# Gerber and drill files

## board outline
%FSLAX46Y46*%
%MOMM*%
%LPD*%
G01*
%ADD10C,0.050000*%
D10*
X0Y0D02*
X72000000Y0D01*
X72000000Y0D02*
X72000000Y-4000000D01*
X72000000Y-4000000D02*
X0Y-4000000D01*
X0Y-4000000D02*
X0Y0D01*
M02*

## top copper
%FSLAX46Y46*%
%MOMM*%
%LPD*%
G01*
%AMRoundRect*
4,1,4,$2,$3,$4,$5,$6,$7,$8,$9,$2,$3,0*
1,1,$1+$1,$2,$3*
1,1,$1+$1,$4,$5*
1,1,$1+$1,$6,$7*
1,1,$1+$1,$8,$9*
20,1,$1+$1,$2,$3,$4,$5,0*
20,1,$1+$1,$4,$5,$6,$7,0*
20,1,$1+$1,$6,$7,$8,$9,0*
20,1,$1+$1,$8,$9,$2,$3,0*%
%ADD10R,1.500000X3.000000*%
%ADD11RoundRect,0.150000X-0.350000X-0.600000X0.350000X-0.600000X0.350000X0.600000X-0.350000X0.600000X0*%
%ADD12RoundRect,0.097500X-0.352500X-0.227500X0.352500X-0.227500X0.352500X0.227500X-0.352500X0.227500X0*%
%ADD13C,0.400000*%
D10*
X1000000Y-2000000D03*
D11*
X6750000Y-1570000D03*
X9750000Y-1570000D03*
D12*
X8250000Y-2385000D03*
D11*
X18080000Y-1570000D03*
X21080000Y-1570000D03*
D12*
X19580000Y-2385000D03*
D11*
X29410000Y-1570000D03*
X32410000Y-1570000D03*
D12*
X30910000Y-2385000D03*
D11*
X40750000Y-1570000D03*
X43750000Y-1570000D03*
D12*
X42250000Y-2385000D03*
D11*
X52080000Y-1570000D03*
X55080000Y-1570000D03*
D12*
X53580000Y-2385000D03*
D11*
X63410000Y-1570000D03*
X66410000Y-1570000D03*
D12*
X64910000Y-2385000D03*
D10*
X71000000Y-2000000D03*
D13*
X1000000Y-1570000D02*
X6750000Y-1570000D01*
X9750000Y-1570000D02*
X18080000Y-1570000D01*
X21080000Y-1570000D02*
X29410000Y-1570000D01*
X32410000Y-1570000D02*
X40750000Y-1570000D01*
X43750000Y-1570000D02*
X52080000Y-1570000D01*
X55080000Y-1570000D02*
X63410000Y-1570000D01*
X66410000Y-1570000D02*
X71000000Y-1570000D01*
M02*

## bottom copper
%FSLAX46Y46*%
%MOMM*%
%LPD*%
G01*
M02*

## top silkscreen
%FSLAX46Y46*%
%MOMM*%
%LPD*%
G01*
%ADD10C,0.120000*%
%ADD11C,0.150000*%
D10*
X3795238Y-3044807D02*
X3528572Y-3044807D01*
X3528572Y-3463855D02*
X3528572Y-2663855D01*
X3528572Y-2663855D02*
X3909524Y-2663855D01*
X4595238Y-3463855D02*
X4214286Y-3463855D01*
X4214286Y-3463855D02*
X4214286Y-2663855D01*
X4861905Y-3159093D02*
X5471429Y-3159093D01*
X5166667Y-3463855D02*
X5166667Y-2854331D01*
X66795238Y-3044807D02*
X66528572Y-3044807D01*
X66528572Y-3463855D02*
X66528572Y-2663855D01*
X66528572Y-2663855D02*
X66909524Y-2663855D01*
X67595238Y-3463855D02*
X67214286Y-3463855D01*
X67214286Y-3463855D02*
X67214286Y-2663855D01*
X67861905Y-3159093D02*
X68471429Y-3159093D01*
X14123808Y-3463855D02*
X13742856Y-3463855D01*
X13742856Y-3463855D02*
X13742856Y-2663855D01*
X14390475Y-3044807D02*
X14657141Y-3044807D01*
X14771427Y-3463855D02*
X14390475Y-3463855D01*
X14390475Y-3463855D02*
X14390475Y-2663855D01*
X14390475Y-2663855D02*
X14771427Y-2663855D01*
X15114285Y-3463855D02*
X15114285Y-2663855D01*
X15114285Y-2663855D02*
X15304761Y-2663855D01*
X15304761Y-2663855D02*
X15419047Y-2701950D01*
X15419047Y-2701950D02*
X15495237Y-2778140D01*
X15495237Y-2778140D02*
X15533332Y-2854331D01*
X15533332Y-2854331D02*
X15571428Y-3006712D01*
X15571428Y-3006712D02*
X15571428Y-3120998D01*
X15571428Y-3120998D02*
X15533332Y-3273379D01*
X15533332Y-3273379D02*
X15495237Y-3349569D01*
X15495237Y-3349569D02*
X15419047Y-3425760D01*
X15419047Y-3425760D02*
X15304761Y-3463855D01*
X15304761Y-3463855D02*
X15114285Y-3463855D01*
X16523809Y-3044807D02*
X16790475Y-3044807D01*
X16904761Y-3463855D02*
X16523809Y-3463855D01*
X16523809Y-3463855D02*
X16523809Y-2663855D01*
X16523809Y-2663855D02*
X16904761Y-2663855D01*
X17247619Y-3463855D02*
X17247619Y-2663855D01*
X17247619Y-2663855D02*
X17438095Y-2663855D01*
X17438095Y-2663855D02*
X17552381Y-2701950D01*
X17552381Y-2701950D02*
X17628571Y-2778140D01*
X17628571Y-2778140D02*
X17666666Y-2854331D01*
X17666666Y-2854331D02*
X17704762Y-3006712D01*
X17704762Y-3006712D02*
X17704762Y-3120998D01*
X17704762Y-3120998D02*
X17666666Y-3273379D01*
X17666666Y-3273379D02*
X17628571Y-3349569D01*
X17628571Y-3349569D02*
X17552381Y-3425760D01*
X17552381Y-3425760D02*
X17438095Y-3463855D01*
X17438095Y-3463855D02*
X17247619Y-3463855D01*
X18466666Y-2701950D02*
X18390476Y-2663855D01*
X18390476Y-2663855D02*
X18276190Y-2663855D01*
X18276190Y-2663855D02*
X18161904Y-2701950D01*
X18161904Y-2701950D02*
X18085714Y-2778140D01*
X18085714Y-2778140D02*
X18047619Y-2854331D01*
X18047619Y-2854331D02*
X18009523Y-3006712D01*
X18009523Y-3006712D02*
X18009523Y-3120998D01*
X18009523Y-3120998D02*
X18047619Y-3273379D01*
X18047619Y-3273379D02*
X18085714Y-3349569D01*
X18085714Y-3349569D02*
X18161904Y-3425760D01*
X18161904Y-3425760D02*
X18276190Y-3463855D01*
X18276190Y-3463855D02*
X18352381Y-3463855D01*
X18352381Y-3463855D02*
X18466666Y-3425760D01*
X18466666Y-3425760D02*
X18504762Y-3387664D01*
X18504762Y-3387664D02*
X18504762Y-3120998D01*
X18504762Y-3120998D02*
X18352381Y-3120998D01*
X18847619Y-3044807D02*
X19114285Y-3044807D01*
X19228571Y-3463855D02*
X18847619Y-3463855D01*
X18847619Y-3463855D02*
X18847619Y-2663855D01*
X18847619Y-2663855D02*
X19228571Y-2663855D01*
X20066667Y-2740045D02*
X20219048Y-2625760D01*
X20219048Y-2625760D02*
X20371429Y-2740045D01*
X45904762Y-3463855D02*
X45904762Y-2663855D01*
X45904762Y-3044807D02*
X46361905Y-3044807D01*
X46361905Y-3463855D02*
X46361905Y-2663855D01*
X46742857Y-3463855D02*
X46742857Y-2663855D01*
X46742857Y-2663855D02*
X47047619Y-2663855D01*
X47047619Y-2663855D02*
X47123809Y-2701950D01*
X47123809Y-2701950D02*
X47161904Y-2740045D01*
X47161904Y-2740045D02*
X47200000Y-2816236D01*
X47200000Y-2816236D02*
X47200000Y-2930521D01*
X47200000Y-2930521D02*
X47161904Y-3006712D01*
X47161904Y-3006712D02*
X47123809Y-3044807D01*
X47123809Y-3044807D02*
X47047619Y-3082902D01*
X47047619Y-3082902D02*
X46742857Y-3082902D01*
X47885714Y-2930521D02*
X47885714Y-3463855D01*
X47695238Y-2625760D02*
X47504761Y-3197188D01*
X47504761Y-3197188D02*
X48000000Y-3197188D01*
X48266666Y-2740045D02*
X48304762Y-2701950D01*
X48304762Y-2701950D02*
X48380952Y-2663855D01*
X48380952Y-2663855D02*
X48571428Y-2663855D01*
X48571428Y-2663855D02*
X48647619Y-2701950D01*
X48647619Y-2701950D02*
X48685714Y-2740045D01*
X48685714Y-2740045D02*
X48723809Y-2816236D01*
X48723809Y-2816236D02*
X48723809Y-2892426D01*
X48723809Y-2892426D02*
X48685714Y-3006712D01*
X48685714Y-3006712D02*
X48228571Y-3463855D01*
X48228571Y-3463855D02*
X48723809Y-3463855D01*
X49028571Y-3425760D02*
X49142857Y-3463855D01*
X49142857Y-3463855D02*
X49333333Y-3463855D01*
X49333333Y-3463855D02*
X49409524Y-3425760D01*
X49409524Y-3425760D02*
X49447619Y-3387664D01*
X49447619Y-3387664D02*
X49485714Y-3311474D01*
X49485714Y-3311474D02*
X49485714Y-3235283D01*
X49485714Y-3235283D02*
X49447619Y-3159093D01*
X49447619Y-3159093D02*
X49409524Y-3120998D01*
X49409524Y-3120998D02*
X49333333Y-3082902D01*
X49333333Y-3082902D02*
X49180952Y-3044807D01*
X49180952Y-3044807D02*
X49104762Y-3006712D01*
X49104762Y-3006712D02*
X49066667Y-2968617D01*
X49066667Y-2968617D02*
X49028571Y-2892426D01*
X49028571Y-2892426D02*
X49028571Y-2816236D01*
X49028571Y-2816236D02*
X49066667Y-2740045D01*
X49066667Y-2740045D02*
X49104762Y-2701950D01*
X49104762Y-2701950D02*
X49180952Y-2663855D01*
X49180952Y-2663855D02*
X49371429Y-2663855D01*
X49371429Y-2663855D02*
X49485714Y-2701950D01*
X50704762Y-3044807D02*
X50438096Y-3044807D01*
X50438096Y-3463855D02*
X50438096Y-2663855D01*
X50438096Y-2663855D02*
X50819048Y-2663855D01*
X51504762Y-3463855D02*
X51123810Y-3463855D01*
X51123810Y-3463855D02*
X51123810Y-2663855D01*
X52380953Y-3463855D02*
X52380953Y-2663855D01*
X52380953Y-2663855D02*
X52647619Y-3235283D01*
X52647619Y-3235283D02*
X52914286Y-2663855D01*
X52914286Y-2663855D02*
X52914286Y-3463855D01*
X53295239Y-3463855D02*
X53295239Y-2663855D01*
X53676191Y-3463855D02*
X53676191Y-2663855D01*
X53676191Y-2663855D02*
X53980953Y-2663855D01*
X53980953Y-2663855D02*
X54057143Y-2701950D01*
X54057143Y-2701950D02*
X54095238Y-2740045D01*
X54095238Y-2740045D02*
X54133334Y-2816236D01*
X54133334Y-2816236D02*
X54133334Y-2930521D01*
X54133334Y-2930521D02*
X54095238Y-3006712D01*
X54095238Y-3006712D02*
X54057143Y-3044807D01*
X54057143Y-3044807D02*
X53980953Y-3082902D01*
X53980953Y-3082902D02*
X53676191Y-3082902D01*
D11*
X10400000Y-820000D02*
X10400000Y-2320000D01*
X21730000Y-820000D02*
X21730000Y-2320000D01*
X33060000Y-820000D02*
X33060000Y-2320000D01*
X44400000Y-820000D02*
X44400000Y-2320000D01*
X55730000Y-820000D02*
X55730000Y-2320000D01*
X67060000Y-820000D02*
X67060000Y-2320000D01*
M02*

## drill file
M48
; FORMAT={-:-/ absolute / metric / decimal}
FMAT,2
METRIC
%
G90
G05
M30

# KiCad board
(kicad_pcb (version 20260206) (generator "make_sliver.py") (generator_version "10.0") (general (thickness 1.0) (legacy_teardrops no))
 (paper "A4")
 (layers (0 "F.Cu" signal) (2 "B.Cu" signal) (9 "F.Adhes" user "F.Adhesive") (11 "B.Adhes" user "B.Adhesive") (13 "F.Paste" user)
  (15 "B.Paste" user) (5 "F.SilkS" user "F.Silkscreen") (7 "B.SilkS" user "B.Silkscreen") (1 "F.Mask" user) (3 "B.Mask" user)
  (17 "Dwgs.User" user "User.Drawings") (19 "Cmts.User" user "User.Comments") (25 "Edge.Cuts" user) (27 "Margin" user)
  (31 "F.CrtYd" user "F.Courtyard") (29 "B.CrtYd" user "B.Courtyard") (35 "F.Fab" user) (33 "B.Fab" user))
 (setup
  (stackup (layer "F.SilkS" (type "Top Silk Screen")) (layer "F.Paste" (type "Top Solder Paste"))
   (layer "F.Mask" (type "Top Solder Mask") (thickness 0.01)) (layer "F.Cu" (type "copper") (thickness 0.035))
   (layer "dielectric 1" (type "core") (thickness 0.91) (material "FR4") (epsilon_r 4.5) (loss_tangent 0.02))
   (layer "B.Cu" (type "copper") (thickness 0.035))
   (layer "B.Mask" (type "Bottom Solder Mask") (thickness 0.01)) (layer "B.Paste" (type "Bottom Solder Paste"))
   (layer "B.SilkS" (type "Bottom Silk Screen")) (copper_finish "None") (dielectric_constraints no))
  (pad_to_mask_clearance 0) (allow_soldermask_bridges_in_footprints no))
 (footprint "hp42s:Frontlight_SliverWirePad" (layer "F.Cu") (at 1 2)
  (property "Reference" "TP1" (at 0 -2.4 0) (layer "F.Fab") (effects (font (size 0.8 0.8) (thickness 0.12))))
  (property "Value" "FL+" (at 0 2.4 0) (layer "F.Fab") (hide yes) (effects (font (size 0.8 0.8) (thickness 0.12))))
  (pad "1" smd rect (at 0 0) (size 1.5 3) (layers "F.Cu" "F.Mask") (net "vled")))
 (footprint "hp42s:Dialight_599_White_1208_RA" (layer "F.Cu") (at 8.25 1.57)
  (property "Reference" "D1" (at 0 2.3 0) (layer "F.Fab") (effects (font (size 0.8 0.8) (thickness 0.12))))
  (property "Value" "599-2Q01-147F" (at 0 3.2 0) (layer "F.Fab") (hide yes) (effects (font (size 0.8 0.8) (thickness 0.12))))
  (fp_line (start 2.15 -0.75) (end 2.15 0.75) (stroke (width 0.15) (type solid)) (layer "F.SilkS"))
  (pad "2" smd roundrect (at -1.5 0) (size 1 1.5) (layers "F.Cu" "F.Paste" "F.Mask") (roundrect_rratio 0.15) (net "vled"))
  (pad "1" smd roundrect (at 1.5 0) (size 1 1.5) (layers "F.Cu" "F.Paste" "F.Mask") (roundrect_rratio 0.15) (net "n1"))
  (pad "3" smd roundrect (at 0 0.815) (size 0.9 0.65) (layers "F.Cu" "F.Paste" "F.Mask") (roundrect_rratio 0.15)))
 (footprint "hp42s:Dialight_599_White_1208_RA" (layer "F.Cu") (at 19.58 1.57)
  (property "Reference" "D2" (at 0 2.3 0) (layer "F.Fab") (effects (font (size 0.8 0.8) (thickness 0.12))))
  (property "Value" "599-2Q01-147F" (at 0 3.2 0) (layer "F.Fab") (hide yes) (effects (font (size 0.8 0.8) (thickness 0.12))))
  (fp_line (start 2.15 -0.75) (end 2.15 0.75) (stroke (width 0.15) (type solid)) (layer "F.SilkS"))
  (pad "2" smd roundrect (at -1.5 0) (size 1 1.5) (layers "F.Cu" "F.Paste" "F.Mask") (roundrect_rratio 0.15) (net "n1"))
  (pad "1" smd roundrect (at 1.5 0) (size 1 1.5) (layers "F.Cu" "F.Paste" "F.Mask") (roundrect_rratio 0.15) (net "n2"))
  (pad "3" smd roundrect (at 0 0.815) (size 0.9 0.65) (layers "F.Cu" "F.Paste" "F.Mask") (roundrect_rratio 0.15)))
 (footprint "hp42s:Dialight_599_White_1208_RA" (layer "F.Cu") (at 30.91 1.57)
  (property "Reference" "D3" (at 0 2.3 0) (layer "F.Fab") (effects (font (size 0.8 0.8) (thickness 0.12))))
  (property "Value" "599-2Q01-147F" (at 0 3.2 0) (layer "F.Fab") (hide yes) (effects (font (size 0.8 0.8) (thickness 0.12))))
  (fp_line (start 2.15 -0.75) (end 2.15 0.75) (stroke (width 0.15) (type solid)) (layer "F.SilkS"))
  (pad "2" smd roundrect (at -1.5 0) (size 1 1.5) (layers "F.Cu" "F.Paste" "F.Mask") (roundrect_rratio 0.15) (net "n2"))
  (pad "1" smd roundrect (at 1.5 0) (size 1 1.5) (layers "F.Cu" "F.Paste" "F.Mask") (roundrect_rratio 0.15) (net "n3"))
  (pad "3" smd roundrect (at 0 0.815) (size 0.9 0.65) (layers "F.Cu" "F.Paste" "F.Mask") (roundrect_rratio 0.15)))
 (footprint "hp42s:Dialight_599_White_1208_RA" (layer "F.Cu") (at 42.25 1.57)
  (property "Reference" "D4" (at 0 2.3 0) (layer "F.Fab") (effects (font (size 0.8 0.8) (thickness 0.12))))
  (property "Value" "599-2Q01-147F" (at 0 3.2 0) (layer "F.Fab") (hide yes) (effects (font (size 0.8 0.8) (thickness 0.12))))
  (fp_line (start 2.15 -0.75) (end 2.15 0.75) (stroke (width 0.15) (type solid)) (layer "F.SilkS"))
  (pad "2" smd roundrect (at -1.5 0) (size 1 1.5) (layers "F.Cu" "F.Paste" "F.Mask") (roundrect_rratio 0.15) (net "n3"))
  (pad "1" smd roundrect (at 1.5 0) (size 1 1.5) (layers "F.Cu" "F.Paste" "F.Mask") (roundrect_rratio 0.15) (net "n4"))
  (pad "3" smd roundrect (at 0 0.815) (size 0.9 0.65) (layers "F.Cu" "F.Paste" "F.Mask") (roundrect_rratio 0.15)))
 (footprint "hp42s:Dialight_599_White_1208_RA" (layer "F.Cu") (at 53.58 1.57)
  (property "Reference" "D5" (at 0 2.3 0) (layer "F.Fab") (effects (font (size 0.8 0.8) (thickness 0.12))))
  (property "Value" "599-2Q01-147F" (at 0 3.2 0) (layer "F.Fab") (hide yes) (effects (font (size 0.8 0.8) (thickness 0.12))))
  (fp_line (start 2.15 -0.75) (end 2.15 0.75) (stroke (width 0.15) (type solid)) (layer "F.SilkS"))
  (pad "2" smd roundrect (at -1.5 0) (size 1 1.5) (layers "F.Cu" "F.Paste" "F.Mask") (roundrect_rratio 0.15) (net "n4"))
  (pad "1" smd roundrect (at 1.5 0) (size 1 1.5) (layers "F.Cu" "F.Paste" "F.Mask") (roundrect_rratio 0.15) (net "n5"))
  (pad "3" smd roundrect (at 0 0.815) (size 0.9 0.65) (layers "F.Cu" "F.Paste" "F.Mask") (roundrect_rratio 0.15)))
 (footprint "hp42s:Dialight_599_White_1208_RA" (layer "F.Cu") (at 64.91 1.57)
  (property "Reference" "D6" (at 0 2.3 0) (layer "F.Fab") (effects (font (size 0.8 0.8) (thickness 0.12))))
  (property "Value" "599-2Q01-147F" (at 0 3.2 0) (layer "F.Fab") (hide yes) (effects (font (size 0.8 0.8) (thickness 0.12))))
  (fp_line (start 2.15 -0.75) (end 2.15 0.75) (stroke (width 0.15) (type solid)) (layer "F.SilkS"))
  (pad "2" smd roundrect (at -1.5 0) (size 1 1.5) (layers "F.Cu" "F.Paste" "F.Mask") (roundrect_rratio 0.15) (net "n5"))
  (pad "1" smd roundrect (at 1.5 0) (size 1 1.5) (layers "F.Cu" "F.Paste" "F.Mask") (roundrect_rratio 0.15) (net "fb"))
  (pad "3" smd roundrect (at 0 0.815) (size 0.9 0.65) (layers "F.Cu" "F.Paste" "F.Mask") (roundrect_rratio 0.15)))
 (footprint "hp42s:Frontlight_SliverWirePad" (layer "F.Cu") (at 71 2)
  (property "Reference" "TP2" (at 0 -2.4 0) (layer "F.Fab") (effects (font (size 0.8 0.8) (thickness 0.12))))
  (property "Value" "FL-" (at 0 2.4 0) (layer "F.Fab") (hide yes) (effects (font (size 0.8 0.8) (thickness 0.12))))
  (pad "1" smd rect (at 0 0) (size 1.5 3) (layers "F.Cu" "F.Mask") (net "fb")))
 (segment (start 1 1.57) (end 6.75 1.57) (width 0.4) (layer "F.Cu") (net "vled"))
 (segment (start 9.75 1.57) (end 18.08 1.57) (width 0.4) (layer "F.Cu") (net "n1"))
 (segment (start 21.08 1.57) (end 29.41 1.57) (width 0.4) (layer "F.Cu") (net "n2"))
 (segment (start 32.41 1.57) (end 40.75 1.57) (width 0.4) (layer "F.Cu") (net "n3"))
 (segment (start 43.75 1.57) (end 52.08 1.57) (width 0.4) (layer "F.Cu") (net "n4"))
 (segment (start 55.08 1.57) (end 63.41 1.57) (width 0.4) (layer "F.Cu") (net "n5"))
 (segment (start 66.41 1.57) (end 71 1.57) (width 0.4) (layer "F.Cu") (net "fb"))
 (gr_line (start 0 0) (end 72 0) (stroke (width 0.05) (type solid)) (layer "Edge.Cuts"))
 (gr_line (start 72 0) (end 72 4) (stroke (width 0.05) (type solid)) (layer "Edge.Cuts"))
 (gr_line (start 72 4) (end 0 4) (stroke (width 0.05) (type solid)) (layer "Edge.Cuts"))
 (gr_line (start 0 4) (end 0 0) (stroke (width 0.05) (type solid)) (layer "Edge.Cuts"))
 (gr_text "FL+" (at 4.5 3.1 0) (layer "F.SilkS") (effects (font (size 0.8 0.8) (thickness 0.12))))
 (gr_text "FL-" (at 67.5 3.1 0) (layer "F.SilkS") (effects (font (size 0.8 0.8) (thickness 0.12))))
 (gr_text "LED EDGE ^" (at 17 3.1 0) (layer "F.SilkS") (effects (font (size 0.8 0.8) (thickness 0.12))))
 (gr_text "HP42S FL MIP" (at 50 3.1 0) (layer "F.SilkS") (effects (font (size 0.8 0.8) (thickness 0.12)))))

